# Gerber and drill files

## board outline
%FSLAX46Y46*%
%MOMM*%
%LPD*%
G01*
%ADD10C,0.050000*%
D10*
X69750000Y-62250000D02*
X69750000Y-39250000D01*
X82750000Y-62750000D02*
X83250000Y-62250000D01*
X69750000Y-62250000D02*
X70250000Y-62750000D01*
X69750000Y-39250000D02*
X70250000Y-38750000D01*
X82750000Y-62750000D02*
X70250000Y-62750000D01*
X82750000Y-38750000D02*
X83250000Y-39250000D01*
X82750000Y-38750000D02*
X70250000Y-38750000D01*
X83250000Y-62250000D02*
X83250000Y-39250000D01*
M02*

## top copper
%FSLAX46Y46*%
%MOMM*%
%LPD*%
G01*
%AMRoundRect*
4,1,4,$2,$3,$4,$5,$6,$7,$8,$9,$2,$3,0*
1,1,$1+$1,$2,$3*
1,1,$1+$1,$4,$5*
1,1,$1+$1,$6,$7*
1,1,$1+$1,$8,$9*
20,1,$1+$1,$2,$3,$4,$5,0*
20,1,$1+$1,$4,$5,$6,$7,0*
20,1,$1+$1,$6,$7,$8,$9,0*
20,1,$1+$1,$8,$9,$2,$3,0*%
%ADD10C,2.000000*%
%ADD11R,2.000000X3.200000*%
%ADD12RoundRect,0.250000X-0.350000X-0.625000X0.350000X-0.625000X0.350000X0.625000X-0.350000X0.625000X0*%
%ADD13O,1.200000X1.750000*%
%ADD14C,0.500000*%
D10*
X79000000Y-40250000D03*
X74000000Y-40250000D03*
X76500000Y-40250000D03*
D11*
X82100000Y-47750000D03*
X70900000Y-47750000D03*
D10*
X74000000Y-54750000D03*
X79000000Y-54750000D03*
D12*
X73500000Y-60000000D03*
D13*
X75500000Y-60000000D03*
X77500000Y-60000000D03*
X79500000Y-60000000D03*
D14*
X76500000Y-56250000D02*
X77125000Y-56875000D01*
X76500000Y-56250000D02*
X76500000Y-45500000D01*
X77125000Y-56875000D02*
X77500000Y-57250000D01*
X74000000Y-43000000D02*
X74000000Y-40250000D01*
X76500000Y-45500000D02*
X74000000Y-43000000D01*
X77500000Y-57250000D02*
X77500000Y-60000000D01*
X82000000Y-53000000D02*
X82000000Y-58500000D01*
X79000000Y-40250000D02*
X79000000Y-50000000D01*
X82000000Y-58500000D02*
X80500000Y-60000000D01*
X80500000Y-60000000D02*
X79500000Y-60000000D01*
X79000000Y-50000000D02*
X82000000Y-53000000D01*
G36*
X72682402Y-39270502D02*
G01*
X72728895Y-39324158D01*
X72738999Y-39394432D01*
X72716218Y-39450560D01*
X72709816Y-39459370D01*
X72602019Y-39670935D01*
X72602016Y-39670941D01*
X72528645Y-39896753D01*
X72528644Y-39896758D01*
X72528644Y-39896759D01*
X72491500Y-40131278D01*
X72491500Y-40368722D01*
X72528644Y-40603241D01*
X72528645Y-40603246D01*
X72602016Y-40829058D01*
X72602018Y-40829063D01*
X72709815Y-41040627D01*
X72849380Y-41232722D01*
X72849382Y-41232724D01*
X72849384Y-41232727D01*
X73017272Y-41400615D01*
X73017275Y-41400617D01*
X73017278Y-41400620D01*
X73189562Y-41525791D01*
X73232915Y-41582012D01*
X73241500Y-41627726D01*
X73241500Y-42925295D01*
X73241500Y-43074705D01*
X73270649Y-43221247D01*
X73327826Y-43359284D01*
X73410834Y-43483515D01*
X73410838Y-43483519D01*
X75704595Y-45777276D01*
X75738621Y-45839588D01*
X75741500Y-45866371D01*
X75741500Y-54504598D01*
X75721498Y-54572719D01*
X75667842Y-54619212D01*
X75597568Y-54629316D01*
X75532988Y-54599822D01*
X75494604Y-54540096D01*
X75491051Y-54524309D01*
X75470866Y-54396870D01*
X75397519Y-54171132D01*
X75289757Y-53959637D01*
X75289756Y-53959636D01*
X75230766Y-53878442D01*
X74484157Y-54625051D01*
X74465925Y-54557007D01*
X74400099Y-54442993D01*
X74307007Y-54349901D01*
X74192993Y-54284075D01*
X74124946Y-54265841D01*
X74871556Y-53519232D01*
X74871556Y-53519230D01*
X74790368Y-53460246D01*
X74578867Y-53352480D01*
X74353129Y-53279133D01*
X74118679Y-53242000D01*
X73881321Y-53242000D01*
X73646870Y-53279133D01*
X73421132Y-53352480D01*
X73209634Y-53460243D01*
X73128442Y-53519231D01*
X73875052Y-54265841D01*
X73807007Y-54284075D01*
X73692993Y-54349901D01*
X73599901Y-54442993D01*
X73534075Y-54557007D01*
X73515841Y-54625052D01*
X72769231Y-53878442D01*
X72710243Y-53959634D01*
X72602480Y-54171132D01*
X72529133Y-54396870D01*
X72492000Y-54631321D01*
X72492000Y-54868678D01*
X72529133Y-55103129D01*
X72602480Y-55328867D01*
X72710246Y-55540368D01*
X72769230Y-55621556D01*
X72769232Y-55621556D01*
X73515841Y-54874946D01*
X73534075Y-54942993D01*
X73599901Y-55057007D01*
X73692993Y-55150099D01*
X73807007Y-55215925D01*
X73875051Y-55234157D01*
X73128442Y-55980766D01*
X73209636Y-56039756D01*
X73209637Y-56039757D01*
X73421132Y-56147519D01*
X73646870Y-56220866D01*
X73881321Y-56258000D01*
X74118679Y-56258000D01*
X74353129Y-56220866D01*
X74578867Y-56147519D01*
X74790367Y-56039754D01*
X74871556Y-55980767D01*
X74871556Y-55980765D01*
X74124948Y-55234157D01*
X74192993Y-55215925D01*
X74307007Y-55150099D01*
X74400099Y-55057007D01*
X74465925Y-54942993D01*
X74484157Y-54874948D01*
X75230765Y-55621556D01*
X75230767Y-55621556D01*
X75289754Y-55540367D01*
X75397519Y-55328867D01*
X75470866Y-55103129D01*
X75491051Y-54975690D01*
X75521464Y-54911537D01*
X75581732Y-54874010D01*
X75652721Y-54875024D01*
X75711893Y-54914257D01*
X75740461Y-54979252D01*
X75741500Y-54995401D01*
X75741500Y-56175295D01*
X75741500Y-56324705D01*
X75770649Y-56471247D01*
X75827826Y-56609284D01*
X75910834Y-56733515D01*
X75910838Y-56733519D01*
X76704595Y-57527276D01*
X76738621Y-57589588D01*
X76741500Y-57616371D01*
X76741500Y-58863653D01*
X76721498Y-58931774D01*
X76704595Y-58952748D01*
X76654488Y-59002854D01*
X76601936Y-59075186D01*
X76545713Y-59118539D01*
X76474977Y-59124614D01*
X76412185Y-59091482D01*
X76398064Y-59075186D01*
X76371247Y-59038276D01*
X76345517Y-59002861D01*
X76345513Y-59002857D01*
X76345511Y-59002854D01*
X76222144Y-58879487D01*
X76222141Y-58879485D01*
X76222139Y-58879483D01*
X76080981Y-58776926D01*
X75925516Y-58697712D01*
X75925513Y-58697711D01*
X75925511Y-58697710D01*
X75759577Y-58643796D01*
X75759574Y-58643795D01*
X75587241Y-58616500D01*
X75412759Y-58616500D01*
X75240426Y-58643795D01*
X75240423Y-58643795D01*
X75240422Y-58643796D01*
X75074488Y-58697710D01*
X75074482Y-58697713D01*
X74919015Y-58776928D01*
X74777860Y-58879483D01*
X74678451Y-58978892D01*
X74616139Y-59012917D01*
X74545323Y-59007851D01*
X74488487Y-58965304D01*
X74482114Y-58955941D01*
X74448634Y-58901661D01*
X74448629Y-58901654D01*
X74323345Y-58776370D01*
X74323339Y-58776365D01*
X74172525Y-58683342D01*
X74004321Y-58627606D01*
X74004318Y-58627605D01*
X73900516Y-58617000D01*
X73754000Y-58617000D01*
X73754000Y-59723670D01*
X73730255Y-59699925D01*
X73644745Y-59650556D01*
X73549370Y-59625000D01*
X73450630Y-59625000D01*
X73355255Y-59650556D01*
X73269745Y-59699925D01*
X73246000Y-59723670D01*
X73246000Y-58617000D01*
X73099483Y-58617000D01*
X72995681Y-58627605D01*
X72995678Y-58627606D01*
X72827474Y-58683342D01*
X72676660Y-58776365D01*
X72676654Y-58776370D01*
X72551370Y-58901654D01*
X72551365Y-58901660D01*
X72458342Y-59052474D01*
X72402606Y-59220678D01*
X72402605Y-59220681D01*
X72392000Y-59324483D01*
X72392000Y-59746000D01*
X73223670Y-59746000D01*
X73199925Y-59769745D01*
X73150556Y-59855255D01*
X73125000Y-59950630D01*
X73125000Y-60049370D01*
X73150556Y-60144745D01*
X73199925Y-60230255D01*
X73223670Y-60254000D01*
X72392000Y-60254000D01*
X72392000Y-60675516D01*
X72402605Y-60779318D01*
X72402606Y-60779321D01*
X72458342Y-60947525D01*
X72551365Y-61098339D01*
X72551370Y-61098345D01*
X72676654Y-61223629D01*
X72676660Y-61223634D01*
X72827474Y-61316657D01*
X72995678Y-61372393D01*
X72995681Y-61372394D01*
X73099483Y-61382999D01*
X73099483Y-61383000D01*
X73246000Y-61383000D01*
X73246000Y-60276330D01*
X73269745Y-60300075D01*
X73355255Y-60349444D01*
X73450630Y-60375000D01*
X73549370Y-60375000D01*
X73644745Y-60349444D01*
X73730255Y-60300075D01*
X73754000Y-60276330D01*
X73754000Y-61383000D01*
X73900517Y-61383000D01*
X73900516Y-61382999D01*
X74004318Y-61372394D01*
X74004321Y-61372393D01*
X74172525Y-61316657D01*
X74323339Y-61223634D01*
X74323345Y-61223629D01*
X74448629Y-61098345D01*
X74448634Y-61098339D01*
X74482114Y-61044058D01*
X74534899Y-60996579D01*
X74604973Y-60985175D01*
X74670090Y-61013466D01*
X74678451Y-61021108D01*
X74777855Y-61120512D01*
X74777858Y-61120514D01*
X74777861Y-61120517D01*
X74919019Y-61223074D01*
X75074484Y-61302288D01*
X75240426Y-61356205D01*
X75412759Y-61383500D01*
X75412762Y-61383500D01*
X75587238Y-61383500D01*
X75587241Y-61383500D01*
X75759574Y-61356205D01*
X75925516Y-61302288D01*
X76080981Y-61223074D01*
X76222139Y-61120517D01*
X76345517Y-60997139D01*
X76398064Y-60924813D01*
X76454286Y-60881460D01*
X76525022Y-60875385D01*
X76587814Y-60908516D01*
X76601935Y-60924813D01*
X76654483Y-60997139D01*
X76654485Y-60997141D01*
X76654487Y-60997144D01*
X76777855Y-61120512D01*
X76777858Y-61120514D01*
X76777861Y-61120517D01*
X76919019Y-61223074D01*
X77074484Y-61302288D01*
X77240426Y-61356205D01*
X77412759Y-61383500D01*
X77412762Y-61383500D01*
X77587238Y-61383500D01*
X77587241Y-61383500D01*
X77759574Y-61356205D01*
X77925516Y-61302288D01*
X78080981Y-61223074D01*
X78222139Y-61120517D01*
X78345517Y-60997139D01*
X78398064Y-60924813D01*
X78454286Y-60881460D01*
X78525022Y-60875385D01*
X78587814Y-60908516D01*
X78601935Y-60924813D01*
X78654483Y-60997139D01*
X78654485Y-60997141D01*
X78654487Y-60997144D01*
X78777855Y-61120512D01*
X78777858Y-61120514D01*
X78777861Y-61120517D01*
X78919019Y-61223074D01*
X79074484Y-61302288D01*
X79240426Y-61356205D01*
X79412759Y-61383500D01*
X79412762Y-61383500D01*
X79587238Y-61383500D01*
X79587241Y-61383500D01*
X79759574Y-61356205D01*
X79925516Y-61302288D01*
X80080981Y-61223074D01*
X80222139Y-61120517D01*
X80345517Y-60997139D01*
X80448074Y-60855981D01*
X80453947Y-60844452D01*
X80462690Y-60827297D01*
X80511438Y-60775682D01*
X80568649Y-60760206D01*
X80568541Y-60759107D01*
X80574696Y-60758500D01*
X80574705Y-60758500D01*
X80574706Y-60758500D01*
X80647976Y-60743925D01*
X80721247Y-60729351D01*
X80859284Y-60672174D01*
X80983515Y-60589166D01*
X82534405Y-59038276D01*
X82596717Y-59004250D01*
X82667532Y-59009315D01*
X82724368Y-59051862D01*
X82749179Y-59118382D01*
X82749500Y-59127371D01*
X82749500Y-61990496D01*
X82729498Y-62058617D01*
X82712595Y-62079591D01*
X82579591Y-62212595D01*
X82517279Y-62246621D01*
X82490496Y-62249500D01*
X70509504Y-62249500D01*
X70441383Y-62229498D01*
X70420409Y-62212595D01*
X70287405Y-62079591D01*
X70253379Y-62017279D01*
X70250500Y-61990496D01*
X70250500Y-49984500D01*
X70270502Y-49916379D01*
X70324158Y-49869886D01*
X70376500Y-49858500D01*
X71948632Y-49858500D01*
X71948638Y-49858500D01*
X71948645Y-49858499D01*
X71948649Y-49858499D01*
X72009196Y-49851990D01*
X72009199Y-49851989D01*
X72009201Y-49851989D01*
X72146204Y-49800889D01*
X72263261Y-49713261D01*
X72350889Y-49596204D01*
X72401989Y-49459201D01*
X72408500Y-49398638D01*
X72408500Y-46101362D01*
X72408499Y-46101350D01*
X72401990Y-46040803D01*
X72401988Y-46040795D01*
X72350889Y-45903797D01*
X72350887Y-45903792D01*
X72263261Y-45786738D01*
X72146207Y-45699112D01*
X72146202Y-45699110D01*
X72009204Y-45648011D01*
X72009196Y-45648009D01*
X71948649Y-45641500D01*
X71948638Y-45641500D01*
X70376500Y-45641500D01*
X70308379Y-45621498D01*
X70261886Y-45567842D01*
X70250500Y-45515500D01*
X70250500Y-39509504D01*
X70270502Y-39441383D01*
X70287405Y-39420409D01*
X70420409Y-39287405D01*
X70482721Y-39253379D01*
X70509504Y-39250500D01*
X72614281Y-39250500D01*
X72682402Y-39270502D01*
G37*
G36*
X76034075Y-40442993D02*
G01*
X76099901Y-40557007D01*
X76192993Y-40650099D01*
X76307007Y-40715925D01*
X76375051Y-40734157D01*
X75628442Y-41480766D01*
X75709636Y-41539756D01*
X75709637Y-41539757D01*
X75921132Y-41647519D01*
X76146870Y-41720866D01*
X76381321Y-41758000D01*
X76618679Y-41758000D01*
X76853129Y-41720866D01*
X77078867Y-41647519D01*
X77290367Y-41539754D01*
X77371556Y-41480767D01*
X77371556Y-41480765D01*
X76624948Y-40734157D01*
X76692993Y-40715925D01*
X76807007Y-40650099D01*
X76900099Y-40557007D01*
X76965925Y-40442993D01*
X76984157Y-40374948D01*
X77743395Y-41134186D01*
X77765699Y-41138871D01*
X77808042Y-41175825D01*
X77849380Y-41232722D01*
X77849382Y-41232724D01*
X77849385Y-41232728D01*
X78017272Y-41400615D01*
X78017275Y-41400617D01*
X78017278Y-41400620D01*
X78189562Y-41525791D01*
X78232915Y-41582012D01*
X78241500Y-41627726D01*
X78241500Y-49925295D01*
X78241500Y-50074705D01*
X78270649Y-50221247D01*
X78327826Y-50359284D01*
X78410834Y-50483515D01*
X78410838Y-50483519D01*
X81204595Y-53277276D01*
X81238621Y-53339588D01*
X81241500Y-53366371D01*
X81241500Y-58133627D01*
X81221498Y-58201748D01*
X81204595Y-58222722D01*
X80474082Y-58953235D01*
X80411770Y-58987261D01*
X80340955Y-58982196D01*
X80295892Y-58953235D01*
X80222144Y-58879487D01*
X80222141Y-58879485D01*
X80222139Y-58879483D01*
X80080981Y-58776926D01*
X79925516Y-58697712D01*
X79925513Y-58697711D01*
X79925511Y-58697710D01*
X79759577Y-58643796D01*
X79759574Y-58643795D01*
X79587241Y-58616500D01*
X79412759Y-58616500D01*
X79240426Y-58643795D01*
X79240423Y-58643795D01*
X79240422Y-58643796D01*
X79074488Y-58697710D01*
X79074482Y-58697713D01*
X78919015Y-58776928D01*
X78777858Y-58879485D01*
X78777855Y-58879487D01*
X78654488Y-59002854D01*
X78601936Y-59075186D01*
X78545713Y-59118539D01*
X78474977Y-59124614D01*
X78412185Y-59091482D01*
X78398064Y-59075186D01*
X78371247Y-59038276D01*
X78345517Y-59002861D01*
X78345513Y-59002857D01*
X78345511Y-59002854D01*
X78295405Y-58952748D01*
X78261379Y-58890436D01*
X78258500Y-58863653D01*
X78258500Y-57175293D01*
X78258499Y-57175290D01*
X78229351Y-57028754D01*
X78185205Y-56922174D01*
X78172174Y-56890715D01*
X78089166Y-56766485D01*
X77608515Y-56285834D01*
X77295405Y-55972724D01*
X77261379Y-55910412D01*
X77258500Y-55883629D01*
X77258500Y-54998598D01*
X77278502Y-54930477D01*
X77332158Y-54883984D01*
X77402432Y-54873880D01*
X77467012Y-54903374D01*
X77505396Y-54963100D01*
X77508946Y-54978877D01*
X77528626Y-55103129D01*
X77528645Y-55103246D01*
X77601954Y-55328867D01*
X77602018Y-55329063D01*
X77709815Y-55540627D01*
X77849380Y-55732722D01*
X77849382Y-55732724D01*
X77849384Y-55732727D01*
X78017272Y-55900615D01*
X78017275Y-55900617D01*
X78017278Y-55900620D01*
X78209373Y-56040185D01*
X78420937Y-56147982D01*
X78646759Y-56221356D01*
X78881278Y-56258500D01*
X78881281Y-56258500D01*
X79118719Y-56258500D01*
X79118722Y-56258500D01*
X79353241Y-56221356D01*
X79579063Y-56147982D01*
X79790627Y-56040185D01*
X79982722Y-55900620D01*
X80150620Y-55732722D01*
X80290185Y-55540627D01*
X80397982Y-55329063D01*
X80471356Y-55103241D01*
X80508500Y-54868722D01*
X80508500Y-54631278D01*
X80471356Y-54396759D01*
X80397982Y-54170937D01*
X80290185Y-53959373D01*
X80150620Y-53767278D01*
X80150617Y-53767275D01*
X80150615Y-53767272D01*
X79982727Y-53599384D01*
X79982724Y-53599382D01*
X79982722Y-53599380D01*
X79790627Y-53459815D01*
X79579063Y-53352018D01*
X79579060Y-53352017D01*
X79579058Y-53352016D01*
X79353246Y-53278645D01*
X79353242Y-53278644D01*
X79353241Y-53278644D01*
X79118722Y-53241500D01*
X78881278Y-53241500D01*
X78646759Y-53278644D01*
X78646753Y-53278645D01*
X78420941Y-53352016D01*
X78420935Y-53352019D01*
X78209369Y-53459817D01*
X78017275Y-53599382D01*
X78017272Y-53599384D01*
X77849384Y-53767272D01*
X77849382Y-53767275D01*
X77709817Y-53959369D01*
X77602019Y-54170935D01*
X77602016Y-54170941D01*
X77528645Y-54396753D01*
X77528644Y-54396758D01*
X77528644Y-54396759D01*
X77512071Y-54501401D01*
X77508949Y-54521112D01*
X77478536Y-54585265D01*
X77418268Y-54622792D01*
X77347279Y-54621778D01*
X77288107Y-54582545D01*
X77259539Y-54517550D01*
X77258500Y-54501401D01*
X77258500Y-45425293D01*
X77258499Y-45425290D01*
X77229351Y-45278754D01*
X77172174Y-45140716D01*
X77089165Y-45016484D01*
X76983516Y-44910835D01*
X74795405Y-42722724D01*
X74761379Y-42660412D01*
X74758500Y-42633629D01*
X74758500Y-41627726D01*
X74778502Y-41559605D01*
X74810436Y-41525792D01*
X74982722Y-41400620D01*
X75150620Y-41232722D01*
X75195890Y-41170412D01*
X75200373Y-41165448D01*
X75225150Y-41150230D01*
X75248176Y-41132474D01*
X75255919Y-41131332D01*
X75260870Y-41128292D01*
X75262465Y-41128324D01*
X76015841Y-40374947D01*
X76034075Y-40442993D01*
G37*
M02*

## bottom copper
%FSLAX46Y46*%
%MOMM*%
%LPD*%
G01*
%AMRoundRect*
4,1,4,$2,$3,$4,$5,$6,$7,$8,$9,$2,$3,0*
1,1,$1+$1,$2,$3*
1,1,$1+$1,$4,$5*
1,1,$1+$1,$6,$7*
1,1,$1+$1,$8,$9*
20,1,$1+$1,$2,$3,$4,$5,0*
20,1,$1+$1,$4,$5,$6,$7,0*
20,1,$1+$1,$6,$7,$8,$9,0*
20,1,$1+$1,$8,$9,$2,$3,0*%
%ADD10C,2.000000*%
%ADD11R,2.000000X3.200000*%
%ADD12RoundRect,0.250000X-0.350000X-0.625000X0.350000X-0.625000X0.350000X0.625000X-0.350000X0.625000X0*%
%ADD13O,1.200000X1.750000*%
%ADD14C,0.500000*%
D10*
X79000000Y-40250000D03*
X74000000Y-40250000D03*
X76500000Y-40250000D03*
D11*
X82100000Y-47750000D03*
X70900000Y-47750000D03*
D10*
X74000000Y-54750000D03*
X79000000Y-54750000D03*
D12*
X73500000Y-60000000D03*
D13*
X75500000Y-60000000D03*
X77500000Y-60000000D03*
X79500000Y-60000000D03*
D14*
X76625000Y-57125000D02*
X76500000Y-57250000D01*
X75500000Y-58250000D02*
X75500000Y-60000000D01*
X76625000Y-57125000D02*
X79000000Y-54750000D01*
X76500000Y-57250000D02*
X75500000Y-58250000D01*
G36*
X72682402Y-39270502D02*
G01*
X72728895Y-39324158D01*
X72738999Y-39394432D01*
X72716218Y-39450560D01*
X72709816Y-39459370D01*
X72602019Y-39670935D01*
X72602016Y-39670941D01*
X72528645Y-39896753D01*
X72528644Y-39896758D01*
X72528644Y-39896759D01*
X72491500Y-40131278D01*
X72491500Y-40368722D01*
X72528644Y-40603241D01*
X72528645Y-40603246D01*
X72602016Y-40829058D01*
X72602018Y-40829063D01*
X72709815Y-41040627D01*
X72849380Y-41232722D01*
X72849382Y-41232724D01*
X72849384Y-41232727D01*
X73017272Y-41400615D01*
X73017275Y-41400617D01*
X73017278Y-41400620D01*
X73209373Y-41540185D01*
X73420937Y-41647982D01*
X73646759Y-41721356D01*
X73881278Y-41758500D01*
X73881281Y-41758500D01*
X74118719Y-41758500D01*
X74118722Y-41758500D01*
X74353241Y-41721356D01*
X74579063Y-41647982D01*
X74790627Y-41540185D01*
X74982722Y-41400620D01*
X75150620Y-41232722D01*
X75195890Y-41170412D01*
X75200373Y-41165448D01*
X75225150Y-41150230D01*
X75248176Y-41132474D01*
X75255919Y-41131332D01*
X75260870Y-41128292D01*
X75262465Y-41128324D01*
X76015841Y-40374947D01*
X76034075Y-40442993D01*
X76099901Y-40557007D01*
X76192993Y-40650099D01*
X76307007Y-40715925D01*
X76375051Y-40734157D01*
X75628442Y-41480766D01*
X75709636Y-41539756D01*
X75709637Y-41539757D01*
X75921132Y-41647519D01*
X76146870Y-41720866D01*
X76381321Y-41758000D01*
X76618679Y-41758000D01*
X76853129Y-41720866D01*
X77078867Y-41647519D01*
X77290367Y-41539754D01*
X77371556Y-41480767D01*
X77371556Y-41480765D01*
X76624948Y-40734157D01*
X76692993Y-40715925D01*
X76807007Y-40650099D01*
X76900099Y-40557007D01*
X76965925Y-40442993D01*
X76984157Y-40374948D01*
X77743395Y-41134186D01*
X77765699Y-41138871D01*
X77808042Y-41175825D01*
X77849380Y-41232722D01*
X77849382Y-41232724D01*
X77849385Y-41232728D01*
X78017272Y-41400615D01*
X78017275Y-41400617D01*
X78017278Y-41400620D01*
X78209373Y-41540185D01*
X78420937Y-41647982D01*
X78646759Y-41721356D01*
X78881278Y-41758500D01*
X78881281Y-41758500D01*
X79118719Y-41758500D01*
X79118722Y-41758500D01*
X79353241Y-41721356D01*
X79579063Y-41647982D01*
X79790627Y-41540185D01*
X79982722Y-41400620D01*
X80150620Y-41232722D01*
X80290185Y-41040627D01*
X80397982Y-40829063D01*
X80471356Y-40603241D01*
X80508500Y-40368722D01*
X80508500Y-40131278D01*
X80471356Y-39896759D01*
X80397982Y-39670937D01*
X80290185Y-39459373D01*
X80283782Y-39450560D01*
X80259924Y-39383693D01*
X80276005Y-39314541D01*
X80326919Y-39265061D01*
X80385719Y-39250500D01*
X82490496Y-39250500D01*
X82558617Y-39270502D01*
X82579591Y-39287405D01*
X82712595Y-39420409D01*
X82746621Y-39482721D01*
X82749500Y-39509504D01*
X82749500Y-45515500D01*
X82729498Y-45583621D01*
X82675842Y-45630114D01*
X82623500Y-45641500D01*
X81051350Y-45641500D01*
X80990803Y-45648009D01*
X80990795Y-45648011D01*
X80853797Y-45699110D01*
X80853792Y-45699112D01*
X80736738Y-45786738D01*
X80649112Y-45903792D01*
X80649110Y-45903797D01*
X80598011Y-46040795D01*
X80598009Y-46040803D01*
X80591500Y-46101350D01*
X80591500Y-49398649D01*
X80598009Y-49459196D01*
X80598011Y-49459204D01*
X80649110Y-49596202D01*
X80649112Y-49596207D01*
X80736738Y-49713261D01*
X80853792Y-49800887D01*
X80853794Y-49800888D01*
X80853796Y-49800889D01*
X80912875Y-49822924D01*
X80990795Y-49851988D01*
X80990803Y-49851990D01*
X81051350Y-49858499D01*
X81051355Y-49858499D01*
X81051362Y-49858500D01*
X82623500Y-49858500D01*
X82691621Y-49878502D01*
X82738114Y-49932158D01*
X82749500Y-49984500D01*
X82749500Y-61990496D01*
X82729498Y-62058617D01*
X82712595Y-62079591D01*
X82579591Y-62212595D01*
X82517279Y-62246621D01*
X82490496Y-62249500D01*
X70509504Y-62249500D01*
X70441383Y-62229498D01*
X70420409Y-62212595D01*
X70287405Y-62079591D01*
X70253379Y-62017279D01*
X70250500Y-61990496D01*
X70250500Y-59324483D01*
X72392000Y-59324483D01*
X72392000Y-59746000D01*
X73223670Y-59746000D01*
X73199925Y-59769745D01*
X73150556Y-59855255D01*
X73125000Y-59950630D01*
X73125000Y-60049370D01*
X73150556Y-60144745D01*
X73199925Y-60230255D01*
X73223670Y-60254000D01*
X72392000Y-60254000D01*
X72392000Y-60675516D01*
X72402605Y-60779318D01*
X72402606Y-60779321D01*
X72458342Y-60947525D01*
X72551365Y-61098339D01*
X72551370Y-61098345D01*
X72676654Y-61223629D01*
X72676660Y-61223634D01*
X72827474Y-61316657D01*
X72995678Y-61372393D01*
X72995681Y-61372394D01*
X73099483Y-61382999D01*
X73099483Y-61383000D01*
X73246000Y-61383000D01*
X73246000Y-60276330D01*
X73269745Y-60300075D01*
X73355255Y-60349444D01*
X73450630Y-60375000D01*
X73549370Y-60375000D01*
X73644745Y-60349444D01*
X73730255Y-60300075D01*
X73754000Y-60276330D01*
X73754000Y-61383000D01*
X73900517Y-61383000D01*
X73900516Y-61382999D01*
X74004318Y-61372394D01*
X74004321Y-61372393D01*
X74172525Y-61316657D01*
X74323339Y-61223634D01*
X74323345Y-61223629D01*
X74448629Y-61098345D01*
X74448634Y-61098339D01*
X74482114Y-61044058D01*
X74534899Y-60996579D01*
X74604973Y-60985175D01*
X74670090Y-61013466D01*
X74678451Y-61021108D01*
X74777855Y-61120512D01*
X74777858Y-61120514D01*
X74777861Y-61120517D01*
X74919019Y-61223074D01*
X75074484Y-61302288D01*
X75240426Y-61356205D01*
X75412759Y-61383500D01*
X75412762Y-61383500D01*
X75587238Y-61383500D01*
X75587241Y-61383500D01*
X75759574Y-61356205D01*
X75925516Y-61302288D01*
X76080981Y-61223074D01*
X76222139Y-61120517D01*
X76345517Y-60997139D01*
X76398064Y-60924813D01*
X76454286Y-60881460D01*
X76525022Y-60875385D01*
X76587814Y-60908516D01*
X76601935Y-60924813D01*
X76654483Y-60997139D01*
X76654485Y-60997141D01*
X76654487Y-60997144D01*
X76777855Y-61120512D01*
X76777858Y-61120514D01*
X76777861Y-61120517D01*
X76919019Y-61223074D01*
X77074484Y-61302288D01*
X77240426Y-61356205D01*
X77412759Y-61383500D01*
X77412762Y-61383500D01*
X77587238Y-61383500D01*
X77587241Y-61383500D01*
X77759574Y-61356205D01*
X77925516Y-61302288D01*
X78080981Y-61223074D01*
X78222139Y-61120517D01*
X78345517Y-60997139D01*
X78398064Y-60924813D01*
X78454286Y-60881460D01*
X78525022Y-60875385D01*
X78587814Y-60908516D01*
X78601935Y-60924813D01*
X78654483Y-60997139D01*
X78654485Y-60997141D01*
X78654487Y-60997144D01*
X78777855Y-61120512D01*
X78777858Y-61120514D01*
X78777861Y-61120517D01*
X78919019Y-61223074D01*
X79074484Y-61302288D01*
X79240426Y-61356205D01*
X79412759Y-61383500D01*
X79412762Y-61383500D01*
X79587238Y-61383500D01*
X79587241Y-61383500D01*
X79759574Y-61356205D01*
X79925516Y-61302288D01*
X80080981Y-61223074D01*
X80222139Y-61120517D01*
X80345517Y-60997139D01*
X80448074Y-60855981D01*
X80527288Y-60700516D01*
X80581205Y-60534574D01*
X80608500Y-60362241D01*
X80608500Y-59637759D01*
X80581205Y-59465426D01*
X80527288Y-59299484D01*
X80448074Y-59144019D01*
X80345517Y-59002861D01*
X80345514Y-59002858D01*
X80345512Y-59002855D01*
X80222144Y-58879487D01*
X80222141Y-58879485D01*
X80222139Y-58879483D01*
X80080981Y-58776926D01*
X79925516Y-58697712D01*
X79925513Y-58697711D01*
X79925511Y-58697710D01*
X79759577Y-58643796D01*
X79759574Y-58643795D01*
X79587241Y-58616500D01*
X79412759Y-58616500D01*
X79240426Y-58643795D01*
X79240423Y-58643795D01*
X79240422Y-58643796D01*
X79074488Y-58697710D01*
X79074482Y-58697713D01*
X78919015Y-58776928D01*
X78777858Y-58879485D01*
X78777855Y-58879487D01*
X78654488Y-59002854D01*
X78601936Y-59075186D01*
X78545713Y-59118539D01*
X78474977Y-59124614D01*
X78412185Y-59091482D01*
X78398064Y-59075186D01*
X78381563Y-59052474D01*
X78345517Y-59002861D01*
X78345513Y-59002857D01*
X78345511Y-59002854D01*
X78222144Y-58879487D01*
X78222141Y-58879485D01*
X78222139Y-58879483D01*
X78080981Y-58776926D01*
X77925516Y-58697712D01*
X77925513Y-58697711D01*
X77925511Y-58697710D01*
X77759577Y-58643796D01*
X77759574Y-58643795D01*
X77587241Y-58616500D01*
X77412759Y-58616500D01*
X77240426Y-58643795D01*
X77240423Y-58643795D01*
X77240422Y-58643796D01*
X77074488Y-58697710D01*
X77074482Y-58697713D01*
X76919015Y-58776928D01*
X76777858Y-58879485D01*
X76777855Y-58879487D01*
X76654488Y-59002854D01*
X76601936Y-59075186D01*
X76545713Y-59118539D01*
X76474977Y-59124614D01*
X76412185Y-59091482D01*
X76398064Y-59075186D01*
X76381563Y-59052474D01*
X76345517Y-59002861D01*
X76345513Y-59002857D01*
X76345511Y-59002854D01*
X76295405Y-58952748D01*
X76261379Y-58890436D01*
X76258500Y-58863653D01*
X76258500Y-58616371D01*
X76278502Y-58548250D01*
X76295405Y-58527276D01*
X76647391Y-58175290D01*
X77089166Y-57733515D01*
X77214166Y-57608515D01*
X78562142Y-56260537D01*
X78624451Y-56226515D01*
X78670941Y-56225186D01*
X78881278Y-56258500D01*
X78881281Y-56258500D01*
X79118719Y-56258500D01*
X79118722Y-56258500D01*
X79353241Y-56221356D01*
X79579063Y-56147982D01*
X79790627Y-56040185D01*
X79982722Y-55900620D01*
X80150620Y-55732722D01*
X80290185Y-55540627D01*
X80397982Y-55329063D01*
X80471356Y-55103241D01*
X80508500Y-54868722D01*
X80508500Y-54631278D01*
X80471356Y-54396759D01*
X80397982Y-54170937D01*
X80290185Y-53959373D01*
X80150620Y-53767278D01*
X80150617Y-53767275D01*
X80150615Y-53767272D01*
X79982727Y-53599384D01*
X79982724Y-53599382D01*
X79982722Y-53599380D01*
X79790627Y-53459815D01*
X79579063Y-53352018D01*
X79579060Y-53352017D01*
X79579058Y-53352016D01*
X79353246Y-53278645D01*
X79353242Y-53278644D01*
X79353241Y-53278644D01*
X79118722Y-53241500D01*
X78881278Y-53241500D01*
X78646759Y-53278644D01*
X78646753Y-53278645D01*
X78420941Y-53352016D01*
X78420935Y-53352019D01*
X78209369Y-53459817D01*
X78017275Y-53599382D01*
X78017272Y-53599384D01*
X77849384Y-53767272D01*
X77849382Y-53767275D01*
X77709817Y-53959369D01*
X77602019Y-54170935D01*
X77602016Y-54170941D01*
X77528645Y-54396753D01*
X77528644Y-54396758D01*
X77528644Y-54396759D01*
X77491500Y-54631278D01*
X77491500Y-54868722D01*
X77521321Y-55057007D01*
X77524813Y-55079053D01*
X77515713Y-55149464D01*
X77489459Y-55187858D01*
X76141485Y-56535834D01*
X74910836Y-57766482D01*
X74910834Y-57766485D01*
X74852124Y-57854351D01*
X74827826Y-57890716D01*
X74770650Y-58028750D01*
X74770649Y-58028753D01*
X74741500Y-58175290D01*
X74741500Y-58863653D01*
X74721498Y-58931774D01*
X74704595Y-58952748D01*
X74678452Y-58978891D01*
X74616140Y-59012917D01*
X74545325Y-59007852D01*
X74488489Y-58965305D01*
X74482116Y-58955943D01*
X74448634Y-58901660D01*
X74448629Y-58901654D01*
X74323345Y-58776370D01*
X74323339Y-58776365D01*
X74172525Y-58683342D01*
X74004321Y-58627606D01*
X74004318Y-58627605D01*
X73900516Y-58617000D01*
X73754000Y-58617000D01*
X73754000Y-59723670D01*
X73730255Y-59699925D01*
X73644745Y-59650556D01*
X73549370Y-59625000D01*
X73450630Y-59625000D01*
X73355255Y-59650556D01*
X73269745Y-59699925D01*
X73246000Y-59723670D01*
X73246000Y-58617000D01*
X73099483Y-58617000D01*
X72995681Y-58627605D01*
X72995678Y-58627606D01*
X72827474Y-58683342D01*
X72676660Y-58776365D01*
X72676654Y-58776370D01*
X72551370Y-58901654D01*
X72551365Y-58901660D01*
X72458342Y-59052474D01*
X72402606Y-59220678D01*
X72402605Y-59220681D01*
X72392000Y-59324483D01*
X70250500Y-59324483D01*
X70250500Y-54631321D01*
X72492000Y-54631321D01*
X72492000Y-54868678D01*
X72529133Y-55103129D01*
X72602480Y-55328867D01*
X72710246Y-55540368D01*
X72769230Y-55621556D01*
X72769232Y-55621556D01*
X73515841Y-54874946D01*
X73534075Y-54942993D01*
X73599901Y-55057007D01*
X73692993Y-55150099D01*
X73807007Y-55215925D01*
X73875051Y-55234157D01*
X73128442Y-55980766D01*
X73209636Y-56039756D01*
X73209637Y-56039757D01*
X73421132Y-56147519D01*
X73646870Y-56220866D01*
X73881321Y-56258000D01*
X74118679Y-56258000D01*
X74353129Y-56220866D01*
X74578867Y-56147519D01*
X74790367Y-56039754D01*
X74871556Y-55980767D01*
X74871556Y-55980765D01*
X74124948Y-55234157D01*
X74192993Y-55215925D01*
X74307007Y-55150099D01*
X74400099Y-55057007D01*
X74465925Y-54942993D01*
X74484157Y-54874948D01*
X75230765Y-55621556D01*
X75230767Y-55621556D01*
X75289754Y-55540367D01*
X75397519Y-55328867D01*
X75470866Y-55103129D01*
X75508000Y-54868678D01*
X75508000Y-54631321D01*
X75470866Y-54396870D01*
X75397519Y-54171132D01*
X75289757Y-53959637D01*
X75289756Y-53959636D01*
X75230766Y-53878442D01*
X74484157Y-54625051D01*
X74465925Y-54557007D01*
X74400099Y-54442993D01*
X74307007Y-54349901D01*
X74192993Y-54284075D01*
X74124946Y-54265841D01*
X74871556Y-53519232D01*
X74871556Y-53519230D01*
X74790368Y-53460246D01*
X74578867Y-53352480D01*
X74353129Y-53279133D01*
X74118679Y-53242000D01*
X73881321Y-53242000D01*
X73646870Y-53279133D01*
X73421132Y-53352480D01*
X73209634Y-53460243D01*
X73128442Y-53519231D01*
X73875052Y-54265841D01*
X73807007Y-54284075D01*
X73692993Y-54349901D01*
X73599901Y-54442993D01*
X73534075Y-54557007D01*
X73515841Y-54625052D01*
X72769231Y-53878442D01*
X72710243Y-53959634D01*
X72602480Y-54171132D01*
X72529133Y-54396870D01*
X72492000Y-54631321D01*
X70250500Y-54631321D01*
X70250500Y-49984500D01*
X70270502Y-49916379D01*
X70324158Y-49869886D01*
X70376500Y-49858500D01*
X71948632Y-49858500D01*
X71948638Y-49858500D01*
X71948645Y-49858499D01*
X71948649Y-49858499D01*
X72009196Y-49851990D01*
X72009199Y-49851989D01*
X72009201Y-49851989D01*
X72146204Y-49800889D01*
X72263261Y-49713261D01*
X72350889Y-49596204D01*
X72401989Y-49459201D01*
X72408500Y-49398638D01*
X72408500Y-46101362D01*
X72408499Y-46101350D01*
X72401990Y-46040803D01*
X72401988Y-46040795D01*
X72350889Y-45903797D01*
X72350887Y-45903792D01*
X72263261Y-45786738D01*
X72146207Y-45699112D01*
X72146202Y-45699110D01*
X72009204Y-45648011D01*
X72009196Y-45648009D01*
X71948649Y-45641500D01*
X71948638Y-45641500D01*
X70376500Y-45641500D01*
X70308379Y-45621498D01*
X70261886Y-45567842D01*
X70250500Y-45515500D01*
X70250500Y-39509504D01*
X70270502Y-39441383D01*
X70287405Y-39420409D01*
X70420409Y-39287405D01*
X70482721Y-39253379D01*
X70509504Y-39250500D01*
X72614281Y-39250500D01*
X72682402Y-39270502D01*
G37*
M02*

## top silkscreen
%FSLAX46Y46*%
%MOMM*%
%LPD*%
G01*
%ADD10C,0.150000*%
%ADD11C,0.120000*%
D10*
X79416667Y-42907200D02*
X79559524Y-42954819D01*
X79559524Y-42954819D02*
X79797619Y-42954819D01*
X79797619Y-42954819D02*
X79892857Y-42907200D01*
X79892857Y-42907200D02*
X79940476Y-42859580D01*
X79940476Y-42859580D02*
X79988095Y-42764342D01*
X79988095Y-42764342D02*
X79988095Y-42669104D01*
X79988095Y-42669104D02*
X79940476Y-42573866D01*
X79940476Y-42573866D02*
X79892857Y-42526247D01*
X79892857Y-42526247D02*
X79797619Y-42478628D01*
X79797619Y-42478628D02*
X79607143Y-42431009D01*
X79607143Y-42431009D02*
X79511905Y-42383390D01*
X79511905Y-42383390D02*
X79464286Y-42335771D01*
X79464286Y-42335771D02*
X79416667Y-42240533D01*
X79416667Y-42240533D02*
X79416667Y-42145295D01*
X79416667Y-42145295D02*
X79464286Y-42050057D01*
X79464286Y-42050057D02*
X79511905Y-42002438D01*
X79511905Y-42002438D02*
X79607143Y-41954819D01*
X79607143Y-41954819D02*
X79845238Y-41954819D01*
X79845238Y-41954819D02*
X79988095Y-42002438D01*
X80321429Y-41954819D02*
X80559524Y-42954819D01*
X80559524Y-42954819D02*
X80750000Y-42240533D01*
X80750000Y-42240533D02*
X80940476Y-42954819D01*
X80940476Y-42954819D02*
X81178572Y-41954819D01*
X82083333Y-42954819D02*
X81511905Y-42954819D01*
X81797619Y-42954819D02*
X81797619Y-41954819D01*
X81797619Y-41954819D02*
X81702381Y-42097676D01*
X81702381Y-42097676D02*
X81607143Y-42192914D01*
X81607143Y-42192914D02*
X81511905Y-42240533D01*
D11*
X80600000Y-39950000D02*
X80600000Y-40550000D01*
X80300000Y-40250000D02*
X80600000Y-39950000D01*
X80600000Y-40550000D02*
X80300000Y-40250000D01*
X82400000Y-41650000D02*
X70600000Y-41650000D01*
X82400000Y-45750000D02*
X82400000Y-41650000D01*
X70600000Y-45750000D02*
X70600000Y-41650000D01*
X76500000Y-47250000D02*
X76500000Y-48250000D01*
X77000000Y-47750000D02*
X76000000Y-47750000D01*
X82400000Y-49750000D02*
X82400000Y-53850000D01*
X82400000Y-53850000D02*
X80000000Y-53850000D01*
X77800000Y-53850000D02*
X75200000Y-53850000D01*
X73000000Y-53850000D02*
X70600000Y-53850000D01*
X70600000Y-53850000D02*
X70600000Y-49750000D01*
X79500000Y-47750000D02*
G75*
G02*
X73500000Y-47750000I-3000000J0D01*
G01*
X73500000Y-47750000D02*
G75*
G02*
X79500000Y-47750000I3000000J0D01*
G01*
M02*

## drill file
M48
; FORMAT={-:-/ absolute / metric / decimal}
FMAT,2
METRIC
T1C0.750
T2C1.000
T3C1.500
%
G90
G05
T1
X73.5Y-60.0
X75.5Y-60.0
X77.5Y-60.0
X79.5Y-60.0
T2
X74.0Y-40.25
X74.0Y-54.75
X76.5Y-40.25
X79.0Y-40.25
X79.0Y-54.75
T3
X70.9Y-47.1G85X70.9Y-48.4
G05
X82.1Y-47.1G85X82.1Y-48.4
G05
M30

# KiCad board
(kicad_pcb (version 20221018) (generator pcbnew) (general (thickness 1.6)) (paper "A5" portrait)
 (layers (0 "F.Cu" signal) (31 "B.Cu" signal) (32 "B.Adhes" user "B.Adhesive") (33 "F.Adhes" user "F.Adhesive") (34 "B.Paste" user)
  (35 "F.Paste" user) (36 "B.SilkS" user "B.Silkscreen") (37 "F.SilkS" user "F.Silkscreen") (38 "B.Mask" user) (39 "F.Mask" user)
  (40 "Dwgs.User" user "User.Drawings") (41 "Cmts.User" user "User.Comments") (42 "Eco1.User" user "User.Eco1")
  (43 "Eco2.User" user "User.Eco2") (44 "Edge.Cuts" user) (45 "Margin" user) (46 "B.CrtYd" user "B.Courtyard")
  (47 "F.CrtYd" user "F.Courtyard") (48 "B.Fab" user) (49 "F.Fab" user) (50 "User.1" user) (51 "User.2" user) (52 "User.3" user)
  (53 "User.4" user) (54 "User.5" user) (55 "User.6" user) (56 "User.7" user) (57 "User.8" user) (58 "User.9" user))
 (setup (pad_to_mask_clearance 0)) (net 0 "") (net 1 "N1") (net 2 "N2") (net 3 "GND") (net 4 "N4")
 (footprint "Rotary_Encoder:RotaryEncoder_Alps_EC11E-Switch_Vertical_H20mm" (layer "F.Cu") (at 79 40.25 -90)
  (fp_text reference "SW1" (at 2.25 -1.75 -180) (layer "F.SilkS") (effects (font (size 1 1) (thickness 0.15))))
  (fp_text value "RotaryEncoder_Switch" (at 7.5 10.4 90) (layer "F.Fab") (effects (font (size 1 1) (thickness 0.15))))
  (fp_line (start -0.3 -1.6) (end 0.3 -1.6) (stroke (width 0.12) (type solid)) (layer "F.SilkS"))
  (fp_line (start 0 -1.3) (end -0.3 -1.6) (stroke (width 0.12) (type solid)) (layer "F.SilkS"))
  (fp_line (start 0.3 -1.6) (end 0 -1.3) (stroke (width 0.12) (type solid)) (layer "F.SilkS"))
  (fp_line (start 1.4 -3.4) (end 1.4 8.4) (stroke (width 0.12) (type solid)) (layer "F.SilkS"))
  (fp_line (start 5.5 -3.4) (end 1.4 -3.4) (stroke (width 0.12) (type solid)) (layer "F.SilkS"))
  (fp_line (start 5.5 8.4) (end 1.4 8.4) (stroke (width 0.12) (type solid)) (layer "F.SilkS"))
  (fp_line (start 7 2.5) (end 8 2.5) (stroke (width 0.12) (type solid)) (layer "F.SilkS"))
  (fp_line (start 7.5 2) (end 7.5 3) (stroke (width 0.12) (type solid)) (layer "F.SilkS"))
  (fp_line (start 9.5 -3.4) (end 13.6 -3.4) (stroke (width 0.12) (type solid)) (layer "F.SilkS"))
  (fp_line (start 13.6 -3.4) (end 13.6 -1) (stroke (width 0.12) (type solid)) (layer "F.SilkS"))
  (fp_line (start 13.6 1.2) (end 13.6 3.8) (stroke (width 0.12) (type solid)) (layer "F.SilkS"))
  (fp_line (start 13.6 6) (end 13.6 8.4) (stroke (width 0.12) (type solid)) (layer "F.SilkS"))
  (fp_line (start 13.6 8.4) (end 9.5 8.4) (stroke (width 0.12) (type solid)) (layer "F.SilkS"))
  (fp_circle (center 7.5 2.5) (end 10.5 2.5) (stroke (width 0.12) (type solid)) (fill none) (layer "F.SilkS"))
  (pad "A" thru_hole circle (at 0 0 270) (size 2 2) (drill 1) (layers "*.Cu" "*.Mask") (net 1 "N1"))
  (pad "B" thru_hole circle (at 0 5 270) (size 2 2) (drill 1) (layers "*.Cu" "*.Mask") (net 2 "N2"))
  (pad "C" thru_hole circle (at 0 2.5 270) (size 2 2) (drill 1) (layers "*.Cu" "*.Mask") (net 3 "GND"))
  (pad "MP" thru_hole rect (at 7.5 -3.1 270) (size 3.2 2) (drill oval 2.8 1.5) (layers "*.Cu" "*.Mask"))
  (pad "MP" thru_hole rect (at 7.5 8.1 270) (size 3.2 2) (drill oval 2.8 1.5) (layers "*.Cu" "*.Mask"))
  (pad "S1" thru_hole circle (at 14.5 5 270) (size 2 2) (drill 1) (layers "*.Cu" "*.Mask") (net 3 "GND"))
  (pad "S2" thru_hole circle (at 14.5 0 270) (size 2 2) (drill 1) (layers "*.Cu" "*.Mask") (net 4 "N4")))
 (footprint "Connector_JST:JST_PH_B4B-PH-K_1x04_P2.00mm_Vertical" (layer "B.Cu") (at 73.5 60)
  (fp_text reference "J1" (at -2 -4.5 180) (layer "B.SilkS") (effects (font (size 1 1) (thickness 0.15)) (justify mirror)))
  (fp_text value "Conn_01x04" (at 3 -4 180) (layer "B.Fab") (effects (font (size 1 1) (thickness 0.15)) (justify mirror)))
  (pad "1" thru_hole roundrect (at 0 0) (size 1.2 1.75) (drill 0.75) (layers "*.Cu" "*.Mask") (roundrect_rratio 0.2083333333) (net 3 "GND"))
  (pad "2" thru_hole oval (at 2 0) (size 1.2 1.75) (drill 0.75) (layers "*.Cu" "*.Mask") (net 4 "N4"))
  (pad "3" thru_hole oval (at 4 0) (size 1.2 1.75) (drill 0.75) (layers "*.Cu" "*.Mask") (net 2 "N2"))
  (pad "4" thru_hole oval (at 6 0) (size 1.2 1.75) (drill 0.75) (layers "*.Cu" "*.Mask") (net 1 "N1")))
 (gr_line (start 69.75 62.25) (end 69.75 39.25) (stroke (width 0.05) (type default)) (layer "Edge.Cuts"))
 (gr_line (start 82.75 62.75) (end 83.25 62.25) (stroke (width 0.05) (type default)) (layer "Edge.Cuts"))
 (gr_line (start 69.75 62.25) (end 70.25 62.75) (stroke (width 0.05) (type default)) (layer "Edge.Cuts"))
 (gr_line (start 69.75 39.25) (end 70.25 38.75) (stroke (width 0.05) (type default)) (layer "Edge.Cuts"))
 (gr_line (start 82.75 62.75) (end 70.25 62.75) (stroke (width 0.05) (type default)) (layer "Edge.Cuts"))
 (gr_line (start 82.75 38.75) (end 83.25 39.25) (stroke (width 0.05) (type default)) (layer "Edge.Cuts"))
 (gr_line (start 82.75 38.75) (end 70.25 38.75) (stroke (width 0.05) (type default)) (layer "Edge.Cuts"))
 (gr_line (start 83.25 62.25) (end 83.25 39.25) (stroke (width 0.05) (type default)) (layer "Edge.Cuts"))
 (segment (start 76.5 56.25) (end 77.125 56.875) (width 0.5) (layer "F.Cu") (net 2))
 (segment (start 76.5 56.25) (end 76.5 45.5) (width 0.5) (layer "F.Cu") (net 2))
 (segment (start 77.125 56.875) (end 77.5 57.25) (width 0.5) (layer "F.Cu") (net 2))
 (segment (start 74 43) (end 74 40.25) (width 0.5) (layer "F.Cu") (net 2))
 (segment (start 76.5 45.5) (end 74 43) (width 0.5) (layer "F.Cu") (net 2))
 (segment (start 77.5 57.25) (end 77.5 60) (width 0.5) (layer "F.Cu") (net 2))
 (segment (start 82 53) (end 82 58.5) (width 0.5) (layer "F.Cu") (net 1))
 (segment (start 79 40.25) (end 79 50) (width 0.5) (layer "F.Cu") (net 1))
 (segment (start 82 58.5) (end 80.5 60) (width 0.5) (layer "F.Cu") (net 1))
 (segment (start 80.5 60) (end 79.5 60) (width 0.5) (layer "F.Cu") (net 1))
 (segment (start 79 50) (end 82 53) (width 0.5) (layer "F.Cu") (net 1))
 (segment (start 76.625 57.125) (end 76.5 57.25) (width 0.5) (layer "B.Cu") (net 4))
 (segment (start 75.5 58.25) (end 75.5 60) (width 0.5) (layer "B.Cu") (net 4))
 (segment (start 76.625 57.125) (end 79 54.75) (width 0.5) (layer "B.Cu") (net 4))
 (segment (start 76.5 57.25) (end 75.5 58.25) (width 0.5) (layer "B.Cu") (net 4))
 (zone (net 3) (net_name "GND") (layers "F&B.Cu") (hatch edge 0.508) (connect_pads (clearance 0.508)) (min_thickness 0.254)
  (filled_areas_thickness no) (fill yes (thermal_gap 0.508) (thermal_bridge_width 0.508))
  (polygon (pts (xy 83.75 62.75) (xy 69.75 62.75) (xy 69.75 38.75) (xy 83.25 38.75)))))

